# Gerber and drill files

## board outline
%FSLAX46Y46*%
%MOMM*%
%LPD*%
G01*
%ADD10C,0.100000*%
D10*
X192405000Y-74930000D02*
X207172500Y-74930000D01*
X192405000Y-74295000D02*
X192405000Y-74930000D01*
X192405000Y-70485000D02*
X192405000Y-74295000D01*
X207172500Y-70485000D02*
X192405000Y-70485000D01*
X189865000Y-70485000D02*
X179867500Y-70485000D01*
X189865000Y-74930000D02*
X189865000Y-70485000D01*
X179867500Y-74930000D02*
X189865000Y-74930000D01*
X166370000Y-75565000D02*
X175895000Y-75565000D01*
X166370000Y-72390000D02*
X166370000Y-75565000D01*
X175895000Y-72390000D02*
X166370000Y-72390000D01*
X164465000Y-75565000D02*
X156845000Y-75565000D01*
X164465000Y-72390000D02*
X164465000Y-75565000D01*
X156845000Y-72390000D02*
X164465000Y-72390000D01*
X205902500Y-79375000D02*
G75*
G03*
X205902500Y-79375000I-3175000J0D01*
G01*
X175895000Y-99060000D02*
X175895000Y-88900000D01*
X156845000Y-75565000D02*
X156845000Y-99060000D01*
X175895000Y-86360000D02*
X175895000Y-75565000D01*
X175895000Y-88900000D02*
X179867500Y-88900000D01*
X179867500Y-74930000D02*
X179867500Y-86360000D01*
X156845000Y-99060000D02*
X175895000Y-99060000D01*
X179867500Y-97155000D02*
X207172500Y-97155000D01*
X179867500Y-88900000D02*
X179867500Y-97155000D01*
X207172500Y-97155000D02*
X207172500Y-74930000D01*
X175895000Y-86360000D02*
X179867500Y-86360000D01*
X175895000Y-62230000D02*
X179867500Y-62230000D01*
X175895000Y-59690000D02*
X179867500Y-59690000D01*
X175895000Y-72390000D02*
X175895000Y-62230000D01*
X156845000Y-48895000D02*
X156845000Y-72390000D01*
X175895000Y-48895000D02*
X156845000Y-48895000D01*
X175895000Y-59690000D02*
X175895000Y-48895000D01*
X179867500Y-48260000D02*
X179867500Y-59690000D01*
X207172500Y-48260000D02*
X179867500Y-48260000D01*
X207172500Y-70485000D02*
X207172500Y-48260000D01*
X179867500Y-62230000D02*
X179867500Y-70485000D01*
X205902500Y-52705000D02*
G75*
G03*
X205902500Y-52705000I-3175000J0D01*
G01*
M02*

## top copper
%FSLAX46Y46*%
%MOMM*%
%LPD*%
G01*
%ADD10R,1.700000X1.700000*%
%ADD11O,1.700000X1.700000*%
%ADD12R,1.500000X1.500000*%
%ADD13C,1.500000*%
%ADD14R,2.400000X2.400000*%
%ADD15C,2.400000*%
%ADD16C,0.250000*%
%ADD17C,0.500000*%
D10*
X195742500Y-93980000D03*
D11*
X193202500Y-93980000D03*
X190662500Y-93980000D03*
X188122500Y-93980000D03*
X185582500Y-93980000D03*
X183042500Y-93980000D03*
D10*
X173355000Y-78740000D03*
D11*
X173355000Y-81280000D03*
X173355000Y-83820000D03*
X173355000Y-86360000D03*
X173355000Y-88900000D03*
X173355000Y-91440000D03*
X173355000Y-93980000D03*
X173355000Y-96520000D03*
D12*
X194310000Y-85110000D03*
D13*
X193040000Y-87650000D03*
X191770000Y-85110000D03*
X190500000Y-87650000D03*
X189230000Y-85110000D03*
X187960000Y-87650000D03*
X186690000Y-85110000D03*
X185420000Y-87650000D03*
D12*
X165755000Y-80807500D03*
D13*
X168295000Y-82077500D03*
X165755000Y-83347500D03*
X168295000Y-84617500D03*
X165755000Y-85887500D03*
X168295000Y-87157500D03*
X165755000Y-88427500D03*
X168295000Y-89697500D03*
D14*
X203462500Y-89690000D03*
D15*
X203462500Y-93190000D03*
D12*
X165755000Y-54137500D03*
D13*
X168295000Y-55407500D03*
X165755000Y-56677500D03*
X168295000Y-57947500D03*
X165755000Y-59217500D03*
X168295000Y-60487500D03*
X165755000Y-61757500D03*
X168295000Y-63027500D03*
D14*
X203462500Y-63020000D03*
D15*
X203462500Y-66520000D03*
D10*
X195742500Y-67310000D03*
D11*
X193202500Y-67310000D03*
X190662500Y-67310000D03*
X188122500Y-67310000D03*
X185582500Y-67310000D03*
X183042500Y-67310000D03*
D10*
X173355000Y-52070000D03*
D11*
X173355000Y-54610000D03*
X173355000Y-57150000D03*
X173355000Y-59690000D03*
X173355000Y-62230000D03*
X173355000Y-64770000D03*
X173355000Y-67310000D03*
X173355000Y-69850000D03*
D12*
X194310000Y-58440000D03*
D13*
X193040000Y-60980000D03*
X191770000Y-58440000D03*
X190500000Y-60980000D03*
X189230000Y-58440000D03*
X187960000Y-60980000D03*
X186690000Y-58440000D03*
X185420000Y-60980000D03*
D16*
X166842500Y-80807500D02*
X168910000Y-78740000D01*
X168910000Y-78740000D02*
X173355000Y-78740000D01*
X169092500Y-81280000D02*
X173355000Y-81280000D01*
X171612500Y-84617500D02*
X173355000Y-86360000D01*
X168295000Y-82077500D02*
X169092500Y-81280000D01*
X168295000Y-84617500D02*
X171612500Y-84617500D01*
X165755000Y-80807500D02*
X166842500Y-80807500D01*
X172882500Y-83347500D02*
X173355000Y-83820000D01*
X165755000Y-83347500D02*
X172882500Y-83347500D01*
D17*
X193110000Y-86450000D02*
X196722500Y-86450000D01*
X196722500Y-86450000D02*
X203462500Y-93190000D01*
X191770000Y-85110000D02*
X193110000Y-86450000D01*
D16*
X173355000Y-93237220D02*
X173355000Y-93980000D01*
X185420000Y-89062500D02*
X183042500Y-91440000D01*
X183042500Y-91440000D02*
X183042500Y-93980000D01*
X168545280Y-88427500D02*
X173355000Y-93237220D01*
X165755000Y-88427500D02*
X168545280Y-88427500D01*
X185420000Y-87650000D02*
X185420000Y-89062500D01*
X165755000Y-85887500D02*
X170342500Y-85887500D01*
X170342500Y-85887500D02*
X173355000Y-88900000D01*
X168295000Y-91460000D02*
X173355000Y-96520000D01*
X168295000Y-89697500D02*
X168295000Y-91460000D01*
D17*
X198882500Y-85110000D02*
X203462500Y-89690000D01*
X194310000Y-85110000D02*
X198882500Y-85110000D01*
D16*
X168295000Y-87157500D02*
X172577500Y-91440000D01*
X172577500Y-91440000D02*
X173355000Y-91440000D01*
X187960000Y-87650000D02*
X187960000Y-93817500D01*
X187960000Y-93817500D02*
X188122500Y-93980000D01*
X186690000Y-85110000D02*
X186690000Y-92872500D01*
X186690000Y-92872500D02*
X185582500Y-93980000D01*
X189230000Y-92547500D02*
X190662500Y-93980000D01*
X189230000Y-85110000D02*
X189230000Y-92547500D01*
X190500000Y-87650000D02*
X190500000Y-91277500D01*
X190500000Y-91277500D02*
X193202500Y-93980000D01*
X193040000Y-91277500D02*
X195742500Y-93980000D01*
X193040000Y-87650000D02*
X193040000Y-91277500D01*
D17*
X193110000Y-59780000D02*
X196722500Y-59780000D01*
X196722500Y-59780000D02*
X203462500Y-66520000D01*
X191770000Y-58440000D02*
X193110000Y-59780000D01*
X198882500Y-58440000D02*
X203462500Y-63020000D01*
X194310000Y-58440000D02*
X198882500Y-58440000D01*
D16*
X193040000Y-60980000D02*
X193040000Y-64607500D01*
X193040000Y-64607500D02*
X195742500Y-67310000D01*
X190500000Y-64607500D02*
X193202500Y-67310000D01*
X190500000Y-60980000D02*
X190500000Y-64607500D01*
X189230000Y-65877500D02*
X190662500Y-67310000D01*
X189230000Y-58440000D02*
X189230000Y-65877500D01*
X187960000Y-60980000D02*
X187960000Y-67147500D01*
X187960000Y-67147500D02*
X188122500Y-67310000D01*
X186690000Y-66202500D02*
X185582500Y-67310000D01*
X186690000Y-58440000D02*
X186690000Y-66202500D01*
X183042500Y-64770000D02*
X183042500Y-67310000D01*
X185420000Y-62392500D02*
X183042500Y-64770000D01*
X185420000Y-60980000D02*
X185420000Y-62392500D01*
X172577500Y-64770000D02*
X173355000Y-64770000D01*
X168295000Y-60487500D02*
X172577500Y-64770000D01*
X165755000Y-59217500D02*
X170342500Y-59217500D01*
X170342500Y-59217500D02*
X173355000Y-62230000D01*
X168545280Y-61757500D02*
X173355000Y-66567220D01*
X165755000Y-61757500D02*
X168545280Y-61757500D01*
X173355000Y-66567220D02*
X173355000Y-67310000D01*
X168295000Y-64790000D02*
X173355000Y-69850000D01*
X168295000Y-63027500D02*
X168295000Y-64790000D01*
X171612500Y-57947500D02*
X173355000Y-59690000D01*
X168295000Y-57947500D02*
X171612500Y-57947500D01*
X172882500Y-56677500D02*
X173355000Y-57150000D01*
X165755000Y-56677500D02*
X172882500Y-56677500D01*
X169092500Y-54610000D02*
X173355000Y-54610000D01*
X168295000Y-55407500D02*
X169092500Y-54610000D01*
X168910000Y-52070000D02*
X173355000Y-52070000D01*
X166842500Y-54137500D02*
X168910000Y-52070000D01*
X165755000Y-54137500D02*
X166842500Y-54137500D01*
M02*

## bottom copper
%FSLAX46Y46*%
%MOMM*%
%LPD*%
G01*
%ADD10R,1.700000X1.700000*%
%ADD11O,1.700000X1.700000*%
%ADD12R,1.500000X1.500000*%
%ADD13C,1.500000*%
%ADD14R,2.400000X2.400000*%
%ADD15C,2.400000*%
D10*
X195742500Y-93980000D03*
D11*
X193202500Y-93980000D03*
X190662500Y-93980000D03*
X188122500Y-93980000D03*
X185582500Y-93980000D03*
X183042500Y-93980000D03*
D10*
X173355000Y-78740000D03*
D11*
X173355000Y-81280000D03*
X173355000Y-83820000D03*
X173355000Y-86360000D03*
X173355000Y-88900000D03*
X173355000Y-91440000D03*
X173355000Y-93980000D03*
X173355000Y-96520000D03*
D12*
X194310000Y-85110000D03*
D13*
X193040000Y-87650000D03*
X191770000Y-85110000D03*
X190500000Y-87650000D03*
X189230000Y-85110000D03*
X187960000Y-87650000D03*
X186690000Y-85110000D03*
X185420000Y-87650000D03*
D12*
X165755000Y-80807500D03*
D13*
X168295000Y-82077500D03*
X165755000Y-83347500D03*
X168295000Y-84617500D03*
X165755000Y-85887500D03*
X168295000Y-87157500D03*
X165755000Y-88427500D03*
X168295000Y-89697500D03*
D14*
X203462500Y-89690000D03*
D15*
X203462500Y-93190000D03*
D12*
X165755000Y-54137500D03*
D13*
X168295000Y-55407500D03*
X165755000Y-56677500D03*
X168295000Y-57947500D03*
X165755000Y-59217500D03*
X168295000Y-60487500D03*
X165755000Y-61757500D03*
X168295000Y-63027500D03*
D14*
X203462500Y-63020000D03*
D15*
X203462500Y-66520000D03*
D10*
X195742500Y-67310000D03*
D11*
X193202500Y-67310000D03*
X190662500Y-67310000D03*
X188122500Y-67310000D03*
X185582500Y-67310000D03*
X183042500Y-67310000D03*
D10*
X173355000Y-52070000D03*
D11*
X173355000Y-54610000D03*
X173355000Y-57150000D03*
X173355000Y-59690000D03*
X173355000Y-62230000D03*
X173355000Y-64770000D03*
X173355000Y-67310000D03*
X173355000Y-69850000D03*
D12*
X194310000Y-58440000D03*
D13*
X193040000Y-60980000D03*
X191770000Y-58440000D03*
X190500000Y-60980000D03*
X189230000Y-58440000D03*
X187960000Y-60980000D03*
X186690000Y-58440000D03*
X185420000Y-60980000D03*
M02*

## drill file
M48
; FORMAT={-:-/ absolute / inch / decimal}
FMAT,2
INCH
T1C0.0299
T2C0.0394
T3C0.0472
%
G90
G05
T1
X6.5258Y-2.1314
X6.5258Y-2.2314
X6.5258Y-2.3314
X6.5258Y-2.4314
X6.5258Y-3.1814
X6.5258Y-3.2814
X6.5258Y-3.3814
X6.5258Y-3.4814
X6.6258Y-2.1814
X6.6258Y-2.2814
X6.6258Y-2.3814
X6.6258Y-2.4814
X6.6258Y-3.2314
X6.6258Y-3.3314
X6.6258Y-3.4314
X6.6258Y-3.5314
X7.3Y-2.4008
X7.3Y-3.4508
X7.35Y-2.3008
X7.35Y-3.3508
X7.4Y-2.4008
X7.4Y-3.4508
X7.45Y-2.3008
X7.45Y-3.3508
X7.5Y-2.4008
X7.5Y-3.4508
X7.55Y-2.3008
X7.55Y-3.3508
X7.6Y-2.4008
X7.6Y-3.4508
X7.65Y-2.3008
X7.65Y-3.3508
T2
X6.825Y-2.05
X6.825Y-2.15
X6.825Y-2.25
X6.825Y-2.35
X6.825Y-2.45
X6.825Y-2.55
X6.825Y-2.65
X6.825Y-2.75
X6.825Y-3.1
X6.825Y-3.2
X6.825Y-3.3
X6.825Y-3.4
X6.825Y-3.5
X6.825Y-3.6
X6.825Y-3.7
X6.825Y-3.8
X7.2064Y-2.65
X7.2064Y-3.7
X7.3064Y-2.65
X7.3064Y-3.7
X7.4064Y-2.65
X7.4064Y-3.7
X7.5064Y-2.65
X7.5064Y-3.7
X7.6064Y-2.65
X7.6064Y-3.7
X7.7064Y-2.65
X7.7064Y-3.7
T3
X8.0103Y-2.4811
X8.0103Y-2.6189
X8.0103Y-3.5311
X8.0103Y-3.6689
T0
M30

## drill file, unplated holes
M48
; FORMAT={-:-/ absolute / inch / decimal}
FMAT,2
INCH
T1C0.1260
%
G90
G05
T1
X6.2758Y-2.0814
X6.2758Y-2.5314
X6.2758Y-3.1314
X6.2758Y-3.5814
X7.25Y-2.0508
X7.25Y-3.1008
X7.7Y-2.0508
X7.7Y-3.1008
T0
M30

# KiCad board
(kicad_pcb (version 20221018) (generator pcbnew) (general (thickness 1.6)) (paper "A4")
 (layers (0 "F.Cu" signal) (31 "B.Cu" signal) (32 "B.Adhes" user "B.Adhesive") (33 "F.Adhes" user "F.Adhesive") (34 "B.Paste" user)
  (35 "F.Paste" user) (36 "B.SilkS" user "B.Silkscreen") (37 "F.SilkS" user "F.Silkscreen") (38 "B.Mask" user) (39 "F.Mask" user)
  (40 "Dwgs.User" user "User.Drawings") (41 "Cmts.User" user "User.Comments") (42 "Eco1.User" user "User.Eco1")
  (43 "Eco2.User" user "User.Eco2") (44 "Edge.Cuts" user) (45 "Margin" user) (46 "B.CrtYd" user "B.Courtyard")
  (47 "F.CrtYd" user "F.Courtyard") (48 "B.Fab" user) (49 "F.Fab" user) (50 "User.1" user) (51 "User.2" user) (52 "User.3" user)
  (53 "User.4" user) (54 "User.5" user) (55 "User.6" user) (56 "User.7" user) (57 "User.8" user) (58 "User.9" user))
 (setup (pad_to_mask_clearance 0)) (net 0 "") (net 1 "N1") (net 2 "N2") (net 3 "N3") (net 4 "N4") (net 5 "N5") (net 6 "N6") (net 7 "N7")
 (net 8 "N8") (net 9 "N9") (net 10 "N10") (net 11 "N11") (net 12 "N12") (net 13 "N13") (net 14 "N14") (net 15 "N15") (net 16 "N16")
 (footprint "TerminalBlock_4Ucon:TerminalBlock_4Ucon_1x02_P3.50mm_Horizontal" (layer "F.Cu") (at 203.4625 89.69 -90)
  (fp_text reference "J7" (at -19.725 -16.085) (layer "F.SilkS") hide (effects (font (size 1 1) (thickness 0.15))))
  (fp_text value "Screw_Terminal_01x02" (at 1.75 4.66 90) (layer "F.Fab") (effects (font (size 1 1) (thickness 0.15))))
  (pad "1" thru_hole rect (at 0 0 270) (size 2.4 2.4) (drill 1.2) (layers "*.Cu" "*.Mask") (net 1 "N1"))
  (pad "2" thru_hole circle (at 3.5 0 270) (size 2.4 2.4) (drill 1.2) (layers "*.Cu" "*.Mask") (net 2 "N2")))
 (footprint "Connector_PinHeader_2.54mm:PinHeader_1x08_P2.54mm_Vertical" (layer "F.Cu") (at 173.355 52.07)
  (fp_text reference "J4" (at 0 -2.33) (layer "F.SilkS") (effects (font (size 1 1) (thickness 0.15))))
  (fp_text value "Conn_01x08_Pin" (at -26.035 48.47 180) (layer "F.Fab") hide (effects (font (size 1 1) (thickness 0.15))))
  (pad "1" thru_hole rect (at 0 0) (size 1.7 1.7) (drill 1) (layers "*.Cu" "*.Mask") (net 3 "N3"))
  (pad "2" thru_hole oval (at 0 2.54) (size 1.7 1.7) (drill 1) (layers "*.Cu" "*.Mask") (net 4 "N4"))
  (pad "3" thru_hole oval (at 0 5.08) (size 1.7 1.7) (drill 1) (layers "*.Cu" "*.Mask") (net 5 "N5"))
  (pad "4" thru_hole oval (at 0 7.62) (size 1.7 1.7) (drill 1) (layers "*.Cu" "*.Mask") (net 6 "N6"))
  (pad "5" thru_hole oval (at 0 10.16) (size 1.7 1.7) (drill 1) (layers "*.Cu" "*.Mask") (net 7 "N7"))
  (pad "6" thru_hole oval (at 0 12.7) (size 1.7 1.7) (drill 1) (layers "*.Cu" "*.Mask") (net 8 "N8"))
  (pad "7" thru_hole oval (at 0 15.24) (size 1.7 1.7) (drill 1) (layers "*.Cu" "*.Mask") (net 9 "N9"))
  (pad "8" thru_hole oval (at 0 17.78) (size 1.7 1.7) (drill 1) (layers "*.Cu" "*.Mask") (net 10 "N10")))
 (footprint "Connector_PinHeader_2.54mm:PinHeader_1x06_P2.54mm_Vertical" (layer "F.Cu") (at 195.7425 93.98 -90)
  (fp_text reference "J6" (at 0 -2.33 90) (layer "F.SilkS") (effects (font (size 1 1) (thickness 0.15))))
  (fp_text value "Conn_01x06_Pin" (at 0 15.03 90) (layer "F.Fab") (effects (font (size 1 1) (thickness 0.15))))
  (pad "1" thru_hole rect (at 0 0 270) (size 1.7 1.7) (drill 1) (layers "*.Cu" "*.Mask") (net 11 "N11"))
  (pad "2" thru_hole oval (at 0 2.54 270) (size 1.7 1.7) (drill 1) (layers "*.Cu" "*.Mask") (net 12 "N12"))
  (pad "3" thru_hole oval (at 0 5.08 270) (size 1.7 1.7) (drill 1) (layers "*.Cu" "*.Mask") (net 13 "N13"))
  (pad "4" thru_hole oval (at 0 7.62 270) (size 1.7 1.7) (drill 1) (layers "*.Cu" "*.Mask") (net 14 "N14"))
  (pad "5" thru_hole oval (at 0 10.16 270) (size 1.7 1.7) (drill 1) (layers "*.Cu" "*.Mask") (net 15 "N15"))
  (pad "6" thru_hole oval (at 0 12.7 270) (size 1.7 1.7) (drill 1) (layers "*.Cu" "*.Mask") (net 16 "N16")))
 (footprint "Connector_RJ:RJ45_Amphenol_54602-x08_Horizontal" (layer "F.Cu") (at 194.31 58.44 180)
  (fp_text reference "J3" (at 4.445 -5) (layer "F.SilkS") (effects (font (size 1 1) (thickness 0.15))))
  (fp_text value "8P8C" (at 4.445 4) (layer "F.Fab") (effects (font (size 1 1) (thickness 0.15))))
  (pad "" np_thru_hole circle (at -1.27 6.35 180) (size 3.2 3.2) (drill 3.2) (layers "*.Cu" "*.Mask"))
  (pad "" np_thru_hole circle (at 10.16 6.35 180) (size 3.2 3.2) (drill 3.2) (layers "*.Cu" "*.Mask"))
  (pad "1" thru_hole rect (at 0 0 180) (size 1.5 1.5) (drill 0.76) (layers "*.Cu" "*.Mask") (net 1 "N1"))
  (pad "2" thru_hole circle (at 1.27 -2.54 180) (size 1.5 1.5) (drill 0.76) (layers "*.Cu" "*.Mask") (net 11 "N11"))
  (pad "3" thru_hole circle (at 2.54 0 180) (size 1.5 1.5) (drill 0.76) (layers "*.Cu" "*.Mask") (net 2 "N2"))
  (pad "4" thru_hole circle (at 3.81 -2.54 180) (size 1.5 1.5) (drill 0.76) (layers "*.Cu" "*.Mask") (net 12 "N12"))
  (pad "5" thru_hole circle (at 5.08 0 180) (size 1.5 1.5) (drill 0.76) (layers "*.Cu" "*.Mask") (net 13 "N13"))
  (pad "6" thru_hole circle (at 6.35 -2.54 180) (size 1.5 1.5) (drill 0.76) (layers "*.Cu" "*.Mask") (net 14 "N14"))
  (pad "7" thru_hole circle (at 7.62 0 180) (size 1.5 1.5) (drill 0.76) (layers "*.Cu" "*.Mask") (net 15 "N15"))
  (pad "8" thru_hole circle (at 8.89 -2.54 180) (size 1.5 1.5) (drill 0.76) (layers "*.Cu" "*.Mask") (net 16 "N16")))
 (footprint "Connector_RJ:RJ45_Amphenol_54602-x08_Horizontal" (layer "F.Cu") (at 165.755 80.8075 -90)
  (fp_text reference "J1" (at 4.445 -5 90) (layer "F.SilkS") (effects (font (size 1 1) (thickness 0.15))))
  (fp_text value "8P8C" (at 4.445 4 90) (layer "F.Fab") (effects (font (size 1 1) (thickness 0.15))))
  (pad "" np_thru_hole circle (at -1.27 6.35 270) (size 3.2 3.2) (drill 3.2) (layers "F&B.Cu" "*.Mask"))
  (pad "" np_thru_hole circle (at 10.16 6.35 270) (size 3.2 3.2) (drill 3.2) (layers "F&B.Cu" "*.Mask"))
  (pad "1" thru_hole rect (at 0 0 270) (size 1.5 1.5) (drill 0.76) (layers "*.Cu" "*.Mask") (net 3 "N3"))
  (pad "2" thru_hole circle (at 1.27 -2.54 270) (size 1.5 1.5) (drill 0.76) (layers "*.Cu" "*.Mask") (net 4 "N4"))
  (pad "3" thru_hole circle (at 2.54 0 270) (size 1.5 1.5) (drill 0.76) (layers "*.Cu" "*.Mask") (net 5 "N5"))
  (pad "4" thru_hole circle (at 3.81 -2.54 270) (size 1.5 1.5) (drill 0.76) (layers "*.Cu" "*.Mask") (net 6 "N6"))
  (pad "5" thru_hole circle (at 5.08 0 270) (size 1.5 1.5) (drill 0.76) (layers "*.Cu" "*.Mask") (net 7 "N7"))
  (pad "6" thru_hole circle (at 6.35 -2.54 270) (size 1.5 1.5) (drill 0.76) (layers "*.Cu" "*.Mask") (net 8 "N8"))
  (pad "7" thru_hole circle (at 7.62 0 270) (size 1.5 1.5) (drill 0.76) (layers "*.Cu" "*.Mask") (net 9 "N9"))
  (pad "8" thru_hole circle (at 8.89 -2.54 270) (size 1.5 1.5) (drill 0.76) (layers "*.Cu" "*.Mask") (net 10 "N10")))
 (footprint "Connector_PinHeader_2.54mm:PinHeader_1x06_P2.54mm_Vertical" (layer "F.Cu") (at 195.7425 67.31 -90)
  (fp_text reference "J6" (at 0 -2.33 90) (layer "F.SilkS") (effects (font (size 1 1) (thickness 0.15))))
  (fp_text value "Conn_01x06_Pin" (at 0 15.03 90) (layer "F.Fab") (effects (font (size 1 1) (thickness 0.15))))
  (pad "1" thru_hole rect (at 0 0 270) (size 1.7 1.7) (drill 1) (layers "*.Cu" "*.Mask") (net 11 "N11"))
  (pad "2" thru_hole oval (at 0 2.54 270) (size 1.7 1.7) (drill 1) (layers "*.Cu" "*.Mask") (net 12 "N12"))
  (pad "3" thru_hole oval (at 0 5.08 270) (size 1.7 1.7) (drill 1) (layers "*.Cu" "*.Mask") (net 13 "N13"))
  (pad "4" thru_hole oval (at 0 7.62 270) (size 1.7 1.7) (drill 1) (layers "*.Cu" "*.Mask") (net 14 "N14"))
  (pad "5" thru_hole oval (at 0 10.16 270) (size 1.7 1.7) (drill 1) (layers "*.Cu" "*.Mask") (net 15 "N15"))
  (pad "6" thru_hole oval (at 0 12.7 270) (size 1.7 1.7) (drill 1) (layers "*.Cu" "*.Mask") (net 16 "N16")))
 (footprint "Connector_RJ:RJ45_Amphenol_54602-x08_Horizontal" (layer "F.Cu") (at 165.755 54.1375 -90)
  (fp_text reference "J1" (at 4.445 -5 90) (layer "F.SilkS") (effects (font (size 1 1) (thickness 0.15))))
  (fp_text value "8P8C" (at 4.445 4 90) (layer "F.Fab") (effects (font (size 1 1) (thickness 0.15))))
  (pad "" np_thru_hole circle (at -1.27 6.35 270) (size 3.2 3.2) (drill 3.2) (layers "*.Cu" "*.Mask"))
  (pad "" np_thru_hole circle (at 10.16 6.35 270) (size 3.2 3.2) (drill 3.2) (layers "*.Cu" "*.Mask"))
  (pad "1" thru_hole rect (at 0 0 270) (size 1.5 1.5) (drill 0.76) (layers "*.Cu" "*.Mask") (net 3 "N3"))
  (pad "2" thru_hole circle (at 1.27 -2.54 270) (size 1.5 1.5) (drill 0.76) (layers "*.Cu" "*.Mask") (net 4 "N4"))
  (pad "3" thru_hole circle (at 2.54 0 270) (size 1.5 1.5) (drill 0.76) (layers "*.Cu" "*.Mask") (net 5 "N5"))
  (pad "4" thru_hole circle (at 3.81 -2.54 270) (size 1.5 1.5) (drill 0.76) (layers "*.Cu" "*.Mask") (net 6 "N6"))
  (pad "5" thru_hole circle (at 5.08 0 270) (size 1.5 1.5) (drill 0.76) (layers "*.Cu" "*.Mask") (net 7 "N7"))
  (pad "6" thru_hole circle (at 6.35 -2.54 270) (size 1.5 1.5) (drill 0.76) (layers "*.Cu" "*.Mask") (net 8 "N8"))
  (pad "7" thru_hole circle (at 7.62 0 270) (size 1.5 1.5) (drill 0.76) (layers "*.Cu" "*.Mask") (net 9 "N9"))
  (pad "8" thru_hole circle (at 8.89 -2.54 270) (size 1.5 1.5) (drill 0.76) (layers "*.Cu" "*.Mask") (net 10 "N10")))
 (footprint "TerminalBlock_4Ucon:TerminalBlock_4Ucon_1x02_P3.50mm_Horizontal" (layer "F.Cu") (at 203.4625 63.02 -90)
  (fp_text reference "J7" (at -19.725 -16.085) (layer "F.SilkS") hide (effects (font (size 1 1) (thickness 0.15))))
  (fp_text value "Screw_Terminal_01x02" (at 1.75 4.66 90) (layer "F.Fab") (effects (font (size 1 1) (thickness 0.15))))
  (pad "1" thru_hole rect (at 0 0 270) (size 2.4 2.4) (drill 1.2) (layers "*.Cu" "*.Mask") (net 1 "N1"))
  (pad "2" thru_hole circle (at 3.5 0 270) (size 2.4 2.4) (drill 1.2) (layers "*.Cu" "*.Mask") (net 2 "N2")))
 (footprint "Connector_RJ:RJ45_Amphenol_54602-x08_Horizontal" (layer "F.Cu") (at 194.31 85.11 180)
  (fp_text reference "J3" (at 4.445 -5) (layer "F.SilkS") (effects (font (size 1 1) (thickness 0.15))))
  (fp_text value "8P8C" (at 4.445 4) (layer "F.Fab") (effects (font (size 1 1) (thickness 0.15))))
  (pad "" np_thru_hole circle (at -1.27 6.35 180) (size 3.2 3.2) (drill 3.2) (layers "F&B.Cu" "*.Mask"))
  (pad "" np_thru_hole circle (at 10.16 6.35 180) (size 3.2 3.2) (drill 3.2) (layers "F&B.Cu" "*.Mask"))
  (pad "1" thru_hole rect (at 0 0 180) (size 1.5 1.5) (drill 0.76) (layers "*.Cu" "*.Mask") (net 1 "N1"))
  (pad "2" thru_hole circle (at 1.27 -2.54 180) (size 1.5 1.5) (drill 0.76) (layers "*.Cu" "*.Mask") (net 11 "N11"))
  (pad "3" thru_hole circle (at 2.54 0 180) (size 1.5 1.5) (drill 0.76) (layers "*.Cu" "*.Mask") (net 2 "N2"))
  (pad "4" thru_hole circle (at 3.81 -2.54 180) (size 1.5 1.5) (drill 0.76) (layers "*.Cu" "*.Mask") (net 12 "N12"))
  (pad "5" thru_hole circle (at 5.08 0 180) (size 1.5 1.5) (drill 0.76) (layers "*.Cu" "*.Mask") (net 13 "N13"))
  (pad "6" thru_hole circle (at 6.35 -2.54 180) (size 1.5 1.5) (drill 0.76) (layers "*.Cu" "*.Mask") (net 14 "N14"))
  (pad "7" thru_hole circle (at 7.62 0 180) (size 1.5 1.5) (drill 0.76) (layers "*.Cu" "*.Mask") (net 15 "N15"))
  (pad "8" thru_hole circle (at 8.89 -2.54 180) (size 1.5 1.5) (drill 0.76) (layers "*.Cu" "*.Mask") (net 16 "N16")))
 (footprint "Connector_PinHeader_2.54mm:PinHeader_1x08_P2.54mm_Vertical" (layer "F.Cu") (at 173.355 78.74)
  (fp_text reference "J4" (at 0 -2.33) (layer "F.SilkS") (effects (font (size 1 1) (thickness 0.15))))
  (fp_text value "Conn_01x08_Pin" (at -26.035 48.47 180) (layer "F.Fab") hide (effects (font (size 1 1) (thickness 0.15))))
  (pad "1" thru_hole rect (at 0 0) (size 1.7 1.7) (drill 1) (layers "*.Cu" "*.Mask") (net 3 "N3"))
  (pad "2" thru_hole oval (at 0 2.54) (size 1.7 1.7) (drill 1) (layers "*.Cu" "*.Mask") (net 4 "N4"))
  (pad "3" thru_hole oval (at 0 5.08) (size 1.7 1.7) (drill 1) (layers "*.Cu" "*.Mask") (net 5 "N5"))
  (pad "4" thru_hole oval (at 0 7.62) (size 1.7 1.7) (drill 1) (layers "*.Cu" "*.Mask") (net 6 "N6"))
  (pad "5" thru_hole oval (at 0 10.16) (size 1.7 1.7) (drill 1) (layers "*.Cu" "*.Mask") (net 7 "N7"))
  (pad "6" thru_hole oval (at 0 12.7) (size 1.7 1.7) (drill 1) (layers "*.Cu" "*.Mask") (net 8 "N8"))
  (pad "7" thru_hole oval (at 0 15.24) (size 1.7 1.7) (drill 1) (layers "*.Cu" "*.Mask") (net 9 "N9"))
  (pad "8" thru_hole oval (at 0 17.78) (size 1.7 1.7) (drill 1) (layers "*.Cu" "*.Mask") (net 10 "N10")))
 (gr_line (start 179.8675 97.155) (end 207.1725 97.155) (stroke (width 0.1) (type default)) (layer "Edge.Cuts"))
 (gr_line (start 175.895 99.06) (end 175.895 88.9) (stroke (width 0.1) (type default)) (layer "Edge.Cuts"))
 (gr_line (start 164.465 72.39) (end 164.465 75.565) (stroke (width 0.1) (type default)) (layer "Edge.Cuts"))
 (gr_line (start 166.37 75.565) (end 175.895 75.565) (stroke (width 0.1) (type default)) (layer "Edge.Cuts"))
 (gr_line (start 166.37 72.39) (end 166.37 75.565) (stroke (width 0.1) (type default)) (layer "Edge.Cuts"))
 (gr_line (start 207.1725 48.26) (end 179.8675 48.26) (stroke (width 0.1) (type default)) (layer "Edge.Cuts"))
 (gr_line (start 179.8675 74.93) (end 189.865 74.93) (stroke (width 0.1) (type default)) (layer "Edge.Cuts"))
 (gr_line (start 156.845 72.39) (end 164.465 72.39) (stroke (width 0.1) (type default)) (layer "Edge.Cuts"))
 (gr_line (start 189.865 74.93) (end 189.865 70.485) (stroke (width 0.1) (type default)) (layer "Edge.Cuts"))
 (gr_line (start 175.895 88.9) (end 179.8675 88.9) (stroke (width 0.1) (type default)) (layer "Edge.Cuts"))
 (gr_line (start 175.895 86.36) (end 179.8675 86.36) (stroke (width 0.1) (type default)) (layer "Edge.Cuts"))
 (gr_circle (center 202.7275 52.705) (end 200.8225 50.165) (stroke (width 0.1) (type default)) (fill none) (layer "Edge.Cuts"))
 (gr_line (start 175.895 59.69) (end 175.895 48.895) (stroke (width 0.1) (type default)) (layer "Edge.Cuts"))
 (gr_line (start 192.405 74.295) (end 192.405 74.93) (stroke (width 0.1) (type default)) (layer "Edge.Cuts"))
 (gr_line (start 175.895 62.23) (end 179.8675 62.23) (stroke (width 0.1) (type default)) (layer "Edge.Cuts"))
 (gr_line (start 179.8675 62.23) (end 179.8675 70.485) (stroke (width 0.1) (type default)) (layer "Edge.Cuts"))
 (gr_line (start 175.895 48.895) (end 156.845 48.895) (stroke (width 0.1) (type default)) (layer "Edge.Cuts"))
 (gr_line (start 175.895 72.39) (end 175.895 62.23) (stroke (width 0.1) (type default)) (layer "Edge.Cuts"))
 (gr_line (start 156.845 75.565) (end 156.845 99.06) (stroke (width 0.1) (type default)) (layer "Edge.Cuts"))
 (gr_line (start 189.865 70.485) (end 179.8675 70.485) (stroke (width 0.1) (type default)) (layer "Edge.Cuts"))
 (gr_line (start 192.405 74.93) (end 207.1725 74.93) (stroke (width 0.1) (type default)) (layer "Edge.Cuts"))
 (gr_line (start 179.8675 88.9) (end 179.8675 97.155) (stroke (width 0.1) (type default)) (layer "Edge.Cuts"))
 (gr_line (start 156.845 48.895) (end 156.845 72.39) (stroke (width 0.1) (type default)) (layer "Edge.Cuts"))
 (gr_line (start 179.8675 48.26) (end 179.8675 59.69) (stroke (width 0.1) (type default)) (layer "Edge.Cuts"))
 (gr_circle (center 202.7275 79.375) (end 200.8225 76.835) (stroke (width 0.1) (type default)) (fill none) (layer "Edge.Cuts"))
 (gr_line (start 175.895 72.39) (end 166.37 72.39) (stroke (width 0.1) (type default)) (layer "Edge.Cuts"))
 (gr_line (start 192.405 70.485) (end 192.405 74.295) (stroke (width 0.1) (type default)) (layer "Edge.Cuts"))
 (gr_line (start 175.895 86.36) (end 175.895 75.565) (stroke (width 0.1) (type default)) (layer "Edge.Cuts"))
 (gr_line (start 207.1725 70.485) (end 192.405 70.485) (stroke (width 0.1) (type default)) (layer "Edge.Cuts"))
 (gr_line (start 179.8675 74.93) (end 179.8675 86.36) (stroke (width 0.1) (type default)) (layer "Edge.Cuts"))
 (gr_line (start 175.895 59.69) (end 179.8675 59.69) (stroke (width 0.1) (type default)) (layer "Edge.Cuts"))
 (gr_line (start 207.1725 70.485) (end 207.1725 48.26) (stroke (width 0.1) (type default)) (layer "Edge.Cuts"))
 (gr_line (start 207.1725 97.155) (end 207.1725 74.93) (stroke (width 0.1) (type default)) (layer "Edge.Cuts"))
 (gr_line (start 164.465 75.565) (end 156.845 75.565) (stroke (width 0.1) (type default)) (layer "Edge.Cuts"))
 (gr_line (start 156.845 99.06) (end 175.895 99.06) (stroke (width 0.1) (type default)) (layer "Edge.Cuts"))
 (segment (start 166.8425 80.8075) (end 168.91 78.74) (width 0.25) (layer "F.Cu") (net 3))
 (segment (start 166.8425 54.1375) (end 168.91 52.07) (width 0.25) (layer "F.Cu") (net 3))
 (segment (start 165.755 54.1375) (end 166.8425 54.1375) (width 0.25) (layer "F.Cu") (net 3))
 (segment (start 168.91 78.74) (end 173.355 78.74) (width 0.25) (layer "F.Cu") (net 3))
 (segment (start 165.755 80.8075) (end 166.8425 80.8075) (width 0.25) (layer "F.Cu") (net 3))
 (segment (start 168.91 52.07) (end 173.355 52.07) (width 0.25) (layer "F.Cu") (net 3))
 (segment (start 169.0925 81.28) (end 173.355 81.28) (width 0.25) (layer "F.Cu") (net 4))
 (segment (start 168.295 55.4075) (end 169.0925 54.61) (width 0.25) (layer "F.Cu") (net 4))
 (segment (start 168.295 82.0775) (end 169.0925 81.28) (width 0.25) (layer "F.Cu") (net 4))
 (segment (start 169.0925 54.61) (end 173.355 54.61) (width 0.25) (layer "F.Cu") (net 4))
 (segment (start 172.8825 56.6775) (end 173.355 57.15) (width 0.25) (layer "F.Cu") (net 5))
 (segment (start 165.755 83.3475) (end 172.8825 83.3475) (width 0.25) (layer "F.Cu") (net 5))
 (segment (start 165.755 56.6775) (end 172.8825 56.6775) (width 0.25) (layer "F.Cu") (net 5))
 (segment (start 172.8825 83.3475) (end 173.355 83.82) (width 0.25) (layer "F.Cu") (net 5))
 (segment (start 171.6125 57.9475) (end 173.355 59.69) (width 0.25) (layer "F.Cu") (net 6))
 (segment (start 171.6125 84.6175) (end 173.355 86.36) (width 0.25) (layer "F.Cu") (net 6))
 (segment (start 168.295 84.6175) (end 171.6125 84.6175) (width 0.25) (layer "F.Cu") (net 6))
 (segment (start 168.295 57.9475) (end 171.6125 57.9475) (width 0.25) (layer "F.Cu") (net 6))
 (segment (start 170.3425 85.8875) (end 173.355 88.9) (width 0.25) (layer "F.Cu") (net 7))
 (segment (start 165.755 85.8875) (end 170.3425 85.8875) (width 0.25) (layer "F.Cu") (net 7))
 (segment (start 165.755 59.2175) (end 170.3425 59.2175) (width 0.25) (layer "F.Cu") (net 7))
 (segment (start 170.3425 59.2175) (end 173.355 62.23) (width 0.25) (layer "F.Cu") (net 7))
 (segment (start 168.295 87.1575) (end 172.5775 91.44) (width 0.25) (layer "F.Cu") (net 8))
 (segment (start 172.5775 91.44) (end 173.355 91.44) (width 0.25) (layer "F.Cu") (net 8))
 (segment (start 168.295 60.4875) (end 172.5775 64.77) (width 0.25) (layer "F.Cu") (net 8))
 (segment (start 172.5775 64.77) (end 173.355 64.77) (width 0.25) (layer "F.Cu") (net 8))
 (segment (start 173.355 66.56722) (end 173.355 67.31) (width 0.25) (layer "F.Cu") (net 9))
 (segment (start 173.355 93.23722) (end 173.355 93.98) (width 0.25) (layer "F.Cu") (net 9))
 (segment (start 165.755 61.7575) (end 168.54528 61.7575) (width 0.25) (layer "F.Cu") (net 9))
 (segment (start 168.54528 61.7575) (end 173.355 66.56722) (width 0.25) (layer "F.Cu") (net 9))
 (segment (start 165.755 88.4275) (end 168.54528 88.4275) (width 0.25) (layer "F.Cu") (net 9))
 (segment (start 168.54528 88.4275) (end 173.355 93.23722) (width 0.25) (layer "F.Cu") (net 9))
 (segment (start 168.295 63.0275) (end 168.295 64.79) (width 0.25) (layer "F.Cu") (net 10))
 (segment (start 168.295 64.79) (end 173.355 69.85) (width 0.25) (layer "F.Cu") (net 10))
 (segment (start 168.295 89.6975) (end 168.295 91.46) (width 0.25) (layer "F.Cu") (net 10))
 (segment (start 168.295 91.46) (end 173.355 96.52) (width 0.25) (layer "F.Cu") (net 10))
 (segment (start 194.31 85.11) (end 198.8825 85.11) (width 0.5) (layer "F.Cu") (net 1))
 (segment (start 198.8825 58.44) (end 203.4625 63.02) (width 0.5) (layer "F.Cu") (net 1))
 (segment (start 194.31 58.44) (end 198.8825 58.44) (width 0.5) (layer "F.Cu") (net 1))
 (segment (start 198.8825 85.11) (end 203.4625 89.69) (width 0.5) (layer "F.Cu") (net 1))
 (segment (start 193.04 60.98) (end 193.04 64.6075) (width 0.25) (layer "F.Cu") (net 11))
 (segment (start 193.04 87.65) (end 193.04 91.2775) (width 0.25) (layer "F.Cu") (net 11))
 (segment (start 193.04 91.2775) (end 195.7425 93.98) (width 0.25) (layer "F.Cu") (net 11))
 (segment (start 193.04 64.6075) (end 195.7425 67.31) (width 0.25) (layer "F.Cu") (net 11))
 (segment (start 191.77 58.44) (end 193.11 59.78) (width 0.5) (layer "F.Cu") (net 2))
 (segment (start 196.7225 86.45) (end 203.4625 93.19) (width 0.5) (layer "F.Cu") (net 2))
 (segment (start 196.7225 59.78) (end 203.4625 66.52) (width 0.5) (layer "F.Cu") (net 2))
 (segment (start 193.11 86.45) (end 196.7225 86.45) (width 0.5) (layer "F.Cu") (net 2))
 (segment (start 191.77 85.11) (end 193.11 86.45) (width 0.5) (layer "F.Cu") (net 2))
 (segment (start 193.11 59.78) (end 196.7225 59.78) (width 0.5) (layer "F.Cu") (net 2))
 (segment (start 190.5 64.6075) (end 193.2025 67.31) (width 0.25) (layer "F.Cu") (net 12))
 (segment (start 190.5 91.2775) (end 193.2025 93.98) (width 0.25) (layer "F.Cu") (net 12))
 (segment (start 190.5 60.98) (end 190.5 64.6075) (width 0.25) (layer "F.Cu") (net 12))
 (segment (start 190.5 87.65) (end 190.5 91.2775) (width 0.25) (layer "F.Cu") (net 12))
 (segment (start 189.23 92.5475) (end 190.6625 93.98) (width 0.25) (layer "F.Cu") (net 13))
 (segment (start 189.23 58.44) (end 189.23 65.8775) (width 0.25) (layer "F.Cu") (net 13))
 (segment (start 189.23 65.8775) (end 190.6625 67.31) (width 0.25) (layer "F.Cu") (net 13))
 (segment (start 189.23 85.11) (end 189.23 92.5475) (width 0.25) (layer "F.Cu") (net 13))
 (segment (start 187.96 60.98) (end 187.96 67.1475) (width 0.25) (layer "F.Cu") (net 14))
 (segment (start 187.96 93.8175) (end 188.1225 93.98) (width 0.25) (layer "F.Cu") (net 14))
 (segment (start 187.96 87.65) (end 187.96 93.8175) (width 0.25) (layer "F.Cu") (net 14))
 (segment (start 187.96 67.1475) (end 188.1225 67.31) (width 0.25) (layer "F.Cu") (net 14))
 (segment (start 186.69 66.2025) (end 185.5825 67.31) (width 0.25) (layer "F.Cu") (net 15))
 (segment (start 186.69 92.8725) (end 185.5825 93.98) (width 0.25) (layer "F.Cu") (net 15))
 (segment (start 186.69 85.11) (end 186.69 92.8725) (width 0.25) (layer "F.Cu") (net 15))
 (segment (start 186.69 58.44) (end 186.69 66.2025) (width 0.25) (layer "F.Cu") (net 15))
 (segment (start 185.42 62.3925) (end 183.0425 64.77) (width 0.25) (layer "F.Cu") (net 16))
 (segment (start 185.42 87.65) (end 185.42 89.0625) (width 0.25) (layer "F.Cu") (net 16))
 (segment (start 183.0425 64.77) (end 183.0425 67.31) (width 0.25) (layer "F.Cu") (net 16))
 (segment (start 183.0425 91.44) (end 183.0425 93.98) (width 0.25) (layer "F.Cu") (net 16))
 (segment (start 185.42 89.0625) (end 183.0425 91.44) (width 0.25) (layer "F.Cu") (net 16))
 (segment (start 185.42 60.98) (end 185.42 62.3925) (width 0.25) (layer "F.Cu") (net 16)))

